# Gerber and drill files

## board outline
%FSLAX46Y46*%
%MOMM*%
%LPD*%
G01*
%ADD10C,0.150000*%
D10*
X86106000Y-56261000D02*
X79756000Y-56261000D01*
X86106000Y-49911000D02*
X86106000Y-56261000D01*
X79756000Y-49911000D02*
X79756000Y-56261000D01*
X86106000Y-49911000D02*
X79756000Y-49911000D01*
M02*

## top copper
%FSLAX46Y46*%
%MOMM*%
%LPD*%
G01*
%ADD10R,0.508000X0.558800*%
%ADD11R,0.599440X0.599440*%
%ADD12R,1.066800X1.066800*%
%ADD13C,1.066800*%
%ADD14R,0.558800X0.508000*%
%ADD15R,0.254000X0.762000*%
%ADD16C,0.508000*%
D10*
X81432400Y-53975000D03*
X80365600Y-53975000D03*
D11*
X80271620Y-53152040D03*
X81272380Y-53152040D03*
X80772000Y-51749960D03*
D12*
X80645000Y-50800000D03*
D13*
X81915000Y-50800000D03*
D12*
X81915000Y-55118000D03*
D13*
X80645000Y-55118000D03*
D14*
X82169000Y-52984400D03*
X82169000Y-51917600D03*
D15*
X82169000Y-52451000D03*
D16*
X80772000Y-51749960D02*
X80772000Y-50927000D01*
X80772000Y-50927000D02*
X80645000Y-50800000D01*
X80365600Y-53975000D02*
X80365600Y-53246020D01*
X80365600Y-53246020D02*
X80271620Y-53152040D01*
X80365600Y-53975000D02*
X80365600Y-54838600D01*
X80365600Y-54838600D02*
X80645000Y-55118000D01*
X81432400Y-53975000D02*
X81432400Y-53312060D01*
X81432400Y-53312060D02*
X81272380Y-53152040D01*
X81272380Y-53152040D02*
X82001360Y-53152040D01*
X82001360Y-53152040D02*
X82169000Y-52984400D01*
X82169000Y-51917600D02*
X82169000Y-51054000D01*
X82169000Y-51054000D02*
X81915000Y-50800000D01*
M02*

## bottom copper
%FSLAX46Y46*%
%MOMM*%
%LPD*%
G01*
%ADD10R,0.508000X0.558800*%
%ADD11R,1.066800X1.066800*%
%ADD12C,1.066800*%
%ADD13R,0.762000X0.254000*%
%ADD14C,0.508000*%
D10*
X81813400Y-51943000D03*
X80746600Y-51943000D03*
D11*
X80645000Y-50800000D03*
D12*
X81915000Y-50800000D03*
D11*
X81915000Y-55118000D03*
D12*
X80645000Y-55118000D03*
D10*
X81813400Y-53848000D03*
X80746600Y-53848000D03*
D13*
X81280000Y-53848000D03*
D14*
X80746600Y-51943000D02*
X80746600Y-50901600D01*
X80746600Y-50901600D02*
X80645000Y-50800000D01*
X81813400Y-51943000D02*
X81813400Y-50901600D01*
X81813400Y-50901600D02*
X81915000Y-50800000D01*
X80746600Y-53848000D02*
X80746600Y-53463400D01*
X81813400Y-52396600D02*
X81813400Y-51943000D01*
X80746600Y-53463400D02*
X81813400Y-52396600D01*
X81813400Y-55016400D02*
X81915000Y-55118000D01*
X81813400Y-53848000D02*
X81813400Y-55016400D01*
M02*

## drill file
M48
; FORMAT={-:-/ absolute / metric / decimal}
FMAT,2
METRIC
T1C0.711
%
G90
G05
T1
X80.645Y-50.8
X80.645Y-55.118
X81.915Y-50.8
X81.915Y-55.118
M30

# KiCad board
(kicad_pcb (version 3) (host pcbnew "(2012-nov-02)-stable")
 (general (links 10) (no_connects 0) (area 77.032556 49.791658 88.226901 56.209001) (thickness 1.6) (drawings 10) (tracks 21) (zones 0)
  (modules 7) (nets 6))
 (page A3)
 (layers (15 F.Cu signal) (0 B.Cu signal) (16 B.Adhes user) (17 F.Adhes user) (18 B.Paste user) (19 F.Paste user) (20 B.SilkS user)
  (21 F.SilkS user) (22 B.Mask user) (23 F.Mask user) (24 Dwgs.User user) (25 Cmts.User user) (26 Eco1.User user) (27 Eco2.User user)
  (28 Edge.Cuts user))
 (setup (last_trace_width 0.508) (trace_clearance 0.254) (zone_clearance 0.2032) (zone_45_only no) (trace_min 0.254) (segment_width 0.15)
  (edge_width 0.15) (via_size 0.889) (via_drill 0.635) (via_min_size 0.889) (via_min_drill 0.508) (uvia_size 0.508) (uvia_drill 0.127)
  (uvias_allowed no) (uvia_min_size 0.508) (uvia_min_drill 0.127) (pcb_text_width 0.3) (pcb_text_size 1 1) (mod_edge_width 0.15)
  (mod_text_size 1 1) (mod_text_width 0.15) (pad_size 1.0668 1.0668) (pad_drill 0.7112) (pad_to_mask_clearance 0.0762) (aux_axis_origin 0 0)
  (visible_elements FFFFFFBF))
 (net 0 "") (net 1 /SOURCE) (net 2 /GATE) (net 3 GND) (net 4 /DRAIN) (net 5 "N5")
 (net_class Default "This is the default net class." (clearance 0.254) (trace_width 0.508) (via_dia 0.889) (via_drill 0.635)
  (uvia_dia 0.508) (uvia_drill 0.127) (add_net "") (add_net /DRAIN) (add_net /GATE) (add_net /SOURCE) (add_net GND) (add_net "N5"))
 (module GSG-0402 (layer F.Cu) (at 80.899 53.975) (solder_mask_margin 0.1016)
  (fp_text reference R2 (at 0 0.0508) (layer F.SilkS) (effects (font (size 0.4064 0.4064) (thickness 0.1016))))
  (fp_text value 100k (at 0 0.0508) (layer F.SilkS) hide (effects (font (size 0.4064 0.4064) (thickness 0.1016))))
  (pad 2 smd rect (at 0.5334 0) (size 0.508 0.5588) (layers F.Cu F.Paste F.Mask) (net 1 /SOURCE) (solder_mask_margin 0.1016))
  (pad 1 smd rect (at -0.5334 0) (size 0.508 0.5588) (layers F.Cu F.Paste F.Mask) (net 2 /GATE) (die_length -2147.483648)
   (solder_mask_margin 0.1016)))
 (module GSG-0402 (layer B.Cu) (at 81.28 51.943) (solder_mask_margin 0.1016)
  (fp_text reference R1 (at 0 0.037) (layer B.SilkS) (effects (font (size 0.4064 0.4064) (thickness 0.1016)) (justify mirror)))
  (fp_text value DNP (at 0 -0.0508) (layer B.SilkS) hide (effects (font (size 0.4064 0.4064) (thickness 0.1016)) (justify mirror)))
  (pad 2 smd rect (at 0.5334 0) (size 0.508 0.5588) (layers B.Cu B.Paste B.Mask) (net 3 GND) (solder_mask_margin 0.1016))
  (pad 1 smd rect (at -0.5334 0) (size 0.508 0.5588) (layers B.Cu B.Paste B.Mask) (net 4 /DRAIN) (die_length -2147.483648)
   (solder_mask_margin 0.1016)))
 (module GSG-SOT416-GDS (layer F.Cu) (at 80.772 52.451)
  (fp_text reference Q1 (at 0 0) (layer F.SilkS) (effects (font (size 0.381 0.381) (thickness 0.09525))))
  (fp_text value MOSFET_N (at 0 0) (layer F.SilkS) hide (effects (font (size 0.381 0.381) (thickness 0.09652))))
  (pad G smd rect (at -0.50038 0.70104) (size 0.59944 0.59944) (layers F.Cu F.Paste F.Mask) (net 2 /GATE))
  (pad S smd rect (at 0.50038 0.70104) (size 0.59944 0.59944) (layers F.Cu F.Paste F.Mask) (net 1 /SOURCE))
  (pad D smd rect (at 0 -0.70104) (size 0.59944 0.59944) (layers F.Cu F.Paste F.Mask) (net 4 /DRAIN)))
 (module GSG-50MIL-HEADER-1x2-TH (layer F.Cu) (at 81.28 50.8)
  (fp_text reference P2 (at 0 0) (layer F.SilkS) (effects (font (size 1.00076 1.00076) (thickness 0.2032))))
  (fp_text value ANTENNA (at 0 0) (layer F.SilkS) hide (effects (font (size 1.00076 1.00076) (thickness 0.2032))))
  (pad 1 thru_hole rect (at -0.635 0) (size 1.0668 1.0668) (drill 0.7112) (layers *.Cu *.Mask) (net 4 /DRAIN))
  (pad 2 thru_hole circle (at 0.635 0) (size 1.0668 1.0668) (drill 0.7112) (layers *.Cu *.Mask) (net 3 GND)))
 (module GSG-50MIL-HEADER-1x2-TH (layer F.Cu) (at 81.28 55.118 180)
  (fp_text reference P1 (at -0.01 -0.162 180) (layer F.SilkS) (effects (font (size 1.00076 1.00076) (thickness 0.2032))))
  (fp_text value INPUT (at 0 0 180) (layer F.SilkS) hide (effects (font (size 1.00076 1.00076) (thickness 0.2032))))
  (pad 1 thru_hole rect (at -0.635 0 180) (size 1.0668 1.0668) (drill 0.7112) (layers *.Cu *.Mask) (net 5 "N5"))
  (pad 2 thru_hole circle (at 0.635 0 180) (size 1.0668 1.0668) (drill 0.7112) (layers *.Cu *.Mask) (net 2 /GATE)))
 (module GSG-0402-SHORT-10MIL (layer B.Cu) (at 81.28 53.848) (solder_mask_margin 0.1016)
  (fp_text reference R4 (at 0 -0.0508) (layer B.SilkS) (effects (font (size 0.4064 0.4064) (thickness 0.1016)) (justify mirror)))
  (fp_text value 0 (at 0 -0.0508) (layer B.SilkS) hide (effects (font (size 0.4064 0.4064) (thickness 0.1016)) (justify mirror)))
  (pad 2 smd rect (at 0.5334 0) (size 0.508 0.5588) (layers B.Cu B.Mask) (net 5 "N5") (solder_mask_margin 0.1016))
  (pad 1 smd rect (at -0.5334 0) (size 0.508 0.5588) (layers B.Cu B.Mask) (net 3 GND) (die_length -2147.483648) (solder_mask_margin 0.1016))
  (pad "" smd rect (at 0 0) (size 0.762 0.254) (layers B.Cu B.Mask)))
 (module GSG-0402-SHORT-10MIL (layer F.Cu) (at 82.169 52.451 270) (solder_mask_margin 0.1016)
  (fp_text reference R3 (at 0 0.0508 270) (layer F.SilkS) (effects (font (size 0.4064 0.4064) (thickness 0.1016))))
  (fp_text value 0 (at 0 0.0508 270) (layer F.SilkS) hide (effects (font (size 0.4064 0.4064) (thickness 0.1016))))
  (pad 2 smd rect (at 0.5334 0 270) (size 0.508 0.5588) (layers F.Cu F.Mask) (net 1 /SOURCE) (solder_mask_margin 0.1016))
  (pad 1 smd rect (at -0.5334 0 270) (size 0.508 0.5588) (layers F.Cu F.Mask) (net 3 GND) (die_length -2147.483648)
   (solder_mask_margin 0.1016))
  (pad "" smd rect (at 0 0 270) (size 0.762 0.254) (layers F.Cu F.Mask)))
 (gr_line (start 86.106 56.261) (end 79.756 56.261) (angle 90) (layer Edge.Cuts) (width 0.15))
 (gr_line (start 86.106 49.911) (end 86.106 56.261) (angle 90) (layer Edge.Cuts) (width 0.15))
 (gr_line (start 79.756 49.911) (end 79.756 56.261) (angle 90) (layer Edge.Cuts) (width 0.15))
 (gr_line (start 86.106 49.911) (end 79.756 49.911) (angle 90) (layer Edge.Cuts) (width 0.15))
 (segment (start 80.7466 51.943) (end 80.7466 50.9016) (width 0.508) (layer B.Cu) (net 4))
 (segment (start 80.7466 50.9016) (end 80.645 50.8) (width 0.508) (layer B.Cu) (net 4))
 (segment (start 80.772 51.74996) (end 80.772 50.927) (width 0.508) (layer F.Cu) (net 4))
 (segment (start 80.772 50.927) (end 80.645 50.8) (width 0.508) (layer F.Cu) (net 4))
 (segment (start 80.3656 53.975) (end 80.3656 53.24602) (width 0.508) (layer F.Cu) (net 2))
 (segment (start 80.3656 53.24602) (end 80.27162 53.15204) (width 0.508) (layer F.Cu) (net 2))
 (segment (start 80.3656 53.975) (end 80.3656 54.8386) (width 0.508) (layer F.Cu) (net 2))
 (segment (start 80.3656 54.8386) (end 80.645 55.118) (width 0.508) (layer F.Cu) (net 2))
 (segment (start 81.4324 53.975) (end 81.4324 53.31206) (width 0.508) (layer F.Cu) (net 1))
 (segment (start 81.4324 53.31206) (end 81.27238 53.15204) (width 0.508) (layer F.Cu) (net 1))
 (segment (start 81.27238 53.15204) (end 82.00136 53.15204) (width 0.508) (layer F.Cu) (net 1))
 (segment (start 82.00136 53.15204) (end 82.169 52.9844) (width 0.508) (layer F.Cu) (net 1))
 (segment (start 81.8134 51.943) (end 81.8134 50.9016) (width 0.508) (layer B.Cu) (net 3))
 (segment (start 81.8134 50.9016) (end 81.915 50.8) (width 0.508) (layer B.Cu) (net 3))
 (segment (start 80.7466 53.848) (end 80.7466 53.4634) (width 0.508) (layer B.Cu) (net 3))
 (segment (start 81.8134 52.3966) (end 81.8134 51.943) (width 0.508) (layer B.Cu) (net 3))
 (segment (start 80.7466 53.4634) (end 81.8134 52.3966) (width 0.508) (layer B.Cu) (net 3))
 (segment (start 82.169 51.9176) (end 82.169 51.054) (width 0.508) (layer F.Cu) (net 3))
 (segment (start 82.169 51.054) (end 81.915 50.8) (width 0.508) (layer F.Cu) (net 3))
 (segment (start 81.8134 55.0164) (end 81.915 55.118) (width 0.508) (layer B.Cu) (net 5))
 (segment (start 81.8134 53.848) (end 81.8134 55.0164) (width 0.508) (layer B.Cu) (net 5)))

